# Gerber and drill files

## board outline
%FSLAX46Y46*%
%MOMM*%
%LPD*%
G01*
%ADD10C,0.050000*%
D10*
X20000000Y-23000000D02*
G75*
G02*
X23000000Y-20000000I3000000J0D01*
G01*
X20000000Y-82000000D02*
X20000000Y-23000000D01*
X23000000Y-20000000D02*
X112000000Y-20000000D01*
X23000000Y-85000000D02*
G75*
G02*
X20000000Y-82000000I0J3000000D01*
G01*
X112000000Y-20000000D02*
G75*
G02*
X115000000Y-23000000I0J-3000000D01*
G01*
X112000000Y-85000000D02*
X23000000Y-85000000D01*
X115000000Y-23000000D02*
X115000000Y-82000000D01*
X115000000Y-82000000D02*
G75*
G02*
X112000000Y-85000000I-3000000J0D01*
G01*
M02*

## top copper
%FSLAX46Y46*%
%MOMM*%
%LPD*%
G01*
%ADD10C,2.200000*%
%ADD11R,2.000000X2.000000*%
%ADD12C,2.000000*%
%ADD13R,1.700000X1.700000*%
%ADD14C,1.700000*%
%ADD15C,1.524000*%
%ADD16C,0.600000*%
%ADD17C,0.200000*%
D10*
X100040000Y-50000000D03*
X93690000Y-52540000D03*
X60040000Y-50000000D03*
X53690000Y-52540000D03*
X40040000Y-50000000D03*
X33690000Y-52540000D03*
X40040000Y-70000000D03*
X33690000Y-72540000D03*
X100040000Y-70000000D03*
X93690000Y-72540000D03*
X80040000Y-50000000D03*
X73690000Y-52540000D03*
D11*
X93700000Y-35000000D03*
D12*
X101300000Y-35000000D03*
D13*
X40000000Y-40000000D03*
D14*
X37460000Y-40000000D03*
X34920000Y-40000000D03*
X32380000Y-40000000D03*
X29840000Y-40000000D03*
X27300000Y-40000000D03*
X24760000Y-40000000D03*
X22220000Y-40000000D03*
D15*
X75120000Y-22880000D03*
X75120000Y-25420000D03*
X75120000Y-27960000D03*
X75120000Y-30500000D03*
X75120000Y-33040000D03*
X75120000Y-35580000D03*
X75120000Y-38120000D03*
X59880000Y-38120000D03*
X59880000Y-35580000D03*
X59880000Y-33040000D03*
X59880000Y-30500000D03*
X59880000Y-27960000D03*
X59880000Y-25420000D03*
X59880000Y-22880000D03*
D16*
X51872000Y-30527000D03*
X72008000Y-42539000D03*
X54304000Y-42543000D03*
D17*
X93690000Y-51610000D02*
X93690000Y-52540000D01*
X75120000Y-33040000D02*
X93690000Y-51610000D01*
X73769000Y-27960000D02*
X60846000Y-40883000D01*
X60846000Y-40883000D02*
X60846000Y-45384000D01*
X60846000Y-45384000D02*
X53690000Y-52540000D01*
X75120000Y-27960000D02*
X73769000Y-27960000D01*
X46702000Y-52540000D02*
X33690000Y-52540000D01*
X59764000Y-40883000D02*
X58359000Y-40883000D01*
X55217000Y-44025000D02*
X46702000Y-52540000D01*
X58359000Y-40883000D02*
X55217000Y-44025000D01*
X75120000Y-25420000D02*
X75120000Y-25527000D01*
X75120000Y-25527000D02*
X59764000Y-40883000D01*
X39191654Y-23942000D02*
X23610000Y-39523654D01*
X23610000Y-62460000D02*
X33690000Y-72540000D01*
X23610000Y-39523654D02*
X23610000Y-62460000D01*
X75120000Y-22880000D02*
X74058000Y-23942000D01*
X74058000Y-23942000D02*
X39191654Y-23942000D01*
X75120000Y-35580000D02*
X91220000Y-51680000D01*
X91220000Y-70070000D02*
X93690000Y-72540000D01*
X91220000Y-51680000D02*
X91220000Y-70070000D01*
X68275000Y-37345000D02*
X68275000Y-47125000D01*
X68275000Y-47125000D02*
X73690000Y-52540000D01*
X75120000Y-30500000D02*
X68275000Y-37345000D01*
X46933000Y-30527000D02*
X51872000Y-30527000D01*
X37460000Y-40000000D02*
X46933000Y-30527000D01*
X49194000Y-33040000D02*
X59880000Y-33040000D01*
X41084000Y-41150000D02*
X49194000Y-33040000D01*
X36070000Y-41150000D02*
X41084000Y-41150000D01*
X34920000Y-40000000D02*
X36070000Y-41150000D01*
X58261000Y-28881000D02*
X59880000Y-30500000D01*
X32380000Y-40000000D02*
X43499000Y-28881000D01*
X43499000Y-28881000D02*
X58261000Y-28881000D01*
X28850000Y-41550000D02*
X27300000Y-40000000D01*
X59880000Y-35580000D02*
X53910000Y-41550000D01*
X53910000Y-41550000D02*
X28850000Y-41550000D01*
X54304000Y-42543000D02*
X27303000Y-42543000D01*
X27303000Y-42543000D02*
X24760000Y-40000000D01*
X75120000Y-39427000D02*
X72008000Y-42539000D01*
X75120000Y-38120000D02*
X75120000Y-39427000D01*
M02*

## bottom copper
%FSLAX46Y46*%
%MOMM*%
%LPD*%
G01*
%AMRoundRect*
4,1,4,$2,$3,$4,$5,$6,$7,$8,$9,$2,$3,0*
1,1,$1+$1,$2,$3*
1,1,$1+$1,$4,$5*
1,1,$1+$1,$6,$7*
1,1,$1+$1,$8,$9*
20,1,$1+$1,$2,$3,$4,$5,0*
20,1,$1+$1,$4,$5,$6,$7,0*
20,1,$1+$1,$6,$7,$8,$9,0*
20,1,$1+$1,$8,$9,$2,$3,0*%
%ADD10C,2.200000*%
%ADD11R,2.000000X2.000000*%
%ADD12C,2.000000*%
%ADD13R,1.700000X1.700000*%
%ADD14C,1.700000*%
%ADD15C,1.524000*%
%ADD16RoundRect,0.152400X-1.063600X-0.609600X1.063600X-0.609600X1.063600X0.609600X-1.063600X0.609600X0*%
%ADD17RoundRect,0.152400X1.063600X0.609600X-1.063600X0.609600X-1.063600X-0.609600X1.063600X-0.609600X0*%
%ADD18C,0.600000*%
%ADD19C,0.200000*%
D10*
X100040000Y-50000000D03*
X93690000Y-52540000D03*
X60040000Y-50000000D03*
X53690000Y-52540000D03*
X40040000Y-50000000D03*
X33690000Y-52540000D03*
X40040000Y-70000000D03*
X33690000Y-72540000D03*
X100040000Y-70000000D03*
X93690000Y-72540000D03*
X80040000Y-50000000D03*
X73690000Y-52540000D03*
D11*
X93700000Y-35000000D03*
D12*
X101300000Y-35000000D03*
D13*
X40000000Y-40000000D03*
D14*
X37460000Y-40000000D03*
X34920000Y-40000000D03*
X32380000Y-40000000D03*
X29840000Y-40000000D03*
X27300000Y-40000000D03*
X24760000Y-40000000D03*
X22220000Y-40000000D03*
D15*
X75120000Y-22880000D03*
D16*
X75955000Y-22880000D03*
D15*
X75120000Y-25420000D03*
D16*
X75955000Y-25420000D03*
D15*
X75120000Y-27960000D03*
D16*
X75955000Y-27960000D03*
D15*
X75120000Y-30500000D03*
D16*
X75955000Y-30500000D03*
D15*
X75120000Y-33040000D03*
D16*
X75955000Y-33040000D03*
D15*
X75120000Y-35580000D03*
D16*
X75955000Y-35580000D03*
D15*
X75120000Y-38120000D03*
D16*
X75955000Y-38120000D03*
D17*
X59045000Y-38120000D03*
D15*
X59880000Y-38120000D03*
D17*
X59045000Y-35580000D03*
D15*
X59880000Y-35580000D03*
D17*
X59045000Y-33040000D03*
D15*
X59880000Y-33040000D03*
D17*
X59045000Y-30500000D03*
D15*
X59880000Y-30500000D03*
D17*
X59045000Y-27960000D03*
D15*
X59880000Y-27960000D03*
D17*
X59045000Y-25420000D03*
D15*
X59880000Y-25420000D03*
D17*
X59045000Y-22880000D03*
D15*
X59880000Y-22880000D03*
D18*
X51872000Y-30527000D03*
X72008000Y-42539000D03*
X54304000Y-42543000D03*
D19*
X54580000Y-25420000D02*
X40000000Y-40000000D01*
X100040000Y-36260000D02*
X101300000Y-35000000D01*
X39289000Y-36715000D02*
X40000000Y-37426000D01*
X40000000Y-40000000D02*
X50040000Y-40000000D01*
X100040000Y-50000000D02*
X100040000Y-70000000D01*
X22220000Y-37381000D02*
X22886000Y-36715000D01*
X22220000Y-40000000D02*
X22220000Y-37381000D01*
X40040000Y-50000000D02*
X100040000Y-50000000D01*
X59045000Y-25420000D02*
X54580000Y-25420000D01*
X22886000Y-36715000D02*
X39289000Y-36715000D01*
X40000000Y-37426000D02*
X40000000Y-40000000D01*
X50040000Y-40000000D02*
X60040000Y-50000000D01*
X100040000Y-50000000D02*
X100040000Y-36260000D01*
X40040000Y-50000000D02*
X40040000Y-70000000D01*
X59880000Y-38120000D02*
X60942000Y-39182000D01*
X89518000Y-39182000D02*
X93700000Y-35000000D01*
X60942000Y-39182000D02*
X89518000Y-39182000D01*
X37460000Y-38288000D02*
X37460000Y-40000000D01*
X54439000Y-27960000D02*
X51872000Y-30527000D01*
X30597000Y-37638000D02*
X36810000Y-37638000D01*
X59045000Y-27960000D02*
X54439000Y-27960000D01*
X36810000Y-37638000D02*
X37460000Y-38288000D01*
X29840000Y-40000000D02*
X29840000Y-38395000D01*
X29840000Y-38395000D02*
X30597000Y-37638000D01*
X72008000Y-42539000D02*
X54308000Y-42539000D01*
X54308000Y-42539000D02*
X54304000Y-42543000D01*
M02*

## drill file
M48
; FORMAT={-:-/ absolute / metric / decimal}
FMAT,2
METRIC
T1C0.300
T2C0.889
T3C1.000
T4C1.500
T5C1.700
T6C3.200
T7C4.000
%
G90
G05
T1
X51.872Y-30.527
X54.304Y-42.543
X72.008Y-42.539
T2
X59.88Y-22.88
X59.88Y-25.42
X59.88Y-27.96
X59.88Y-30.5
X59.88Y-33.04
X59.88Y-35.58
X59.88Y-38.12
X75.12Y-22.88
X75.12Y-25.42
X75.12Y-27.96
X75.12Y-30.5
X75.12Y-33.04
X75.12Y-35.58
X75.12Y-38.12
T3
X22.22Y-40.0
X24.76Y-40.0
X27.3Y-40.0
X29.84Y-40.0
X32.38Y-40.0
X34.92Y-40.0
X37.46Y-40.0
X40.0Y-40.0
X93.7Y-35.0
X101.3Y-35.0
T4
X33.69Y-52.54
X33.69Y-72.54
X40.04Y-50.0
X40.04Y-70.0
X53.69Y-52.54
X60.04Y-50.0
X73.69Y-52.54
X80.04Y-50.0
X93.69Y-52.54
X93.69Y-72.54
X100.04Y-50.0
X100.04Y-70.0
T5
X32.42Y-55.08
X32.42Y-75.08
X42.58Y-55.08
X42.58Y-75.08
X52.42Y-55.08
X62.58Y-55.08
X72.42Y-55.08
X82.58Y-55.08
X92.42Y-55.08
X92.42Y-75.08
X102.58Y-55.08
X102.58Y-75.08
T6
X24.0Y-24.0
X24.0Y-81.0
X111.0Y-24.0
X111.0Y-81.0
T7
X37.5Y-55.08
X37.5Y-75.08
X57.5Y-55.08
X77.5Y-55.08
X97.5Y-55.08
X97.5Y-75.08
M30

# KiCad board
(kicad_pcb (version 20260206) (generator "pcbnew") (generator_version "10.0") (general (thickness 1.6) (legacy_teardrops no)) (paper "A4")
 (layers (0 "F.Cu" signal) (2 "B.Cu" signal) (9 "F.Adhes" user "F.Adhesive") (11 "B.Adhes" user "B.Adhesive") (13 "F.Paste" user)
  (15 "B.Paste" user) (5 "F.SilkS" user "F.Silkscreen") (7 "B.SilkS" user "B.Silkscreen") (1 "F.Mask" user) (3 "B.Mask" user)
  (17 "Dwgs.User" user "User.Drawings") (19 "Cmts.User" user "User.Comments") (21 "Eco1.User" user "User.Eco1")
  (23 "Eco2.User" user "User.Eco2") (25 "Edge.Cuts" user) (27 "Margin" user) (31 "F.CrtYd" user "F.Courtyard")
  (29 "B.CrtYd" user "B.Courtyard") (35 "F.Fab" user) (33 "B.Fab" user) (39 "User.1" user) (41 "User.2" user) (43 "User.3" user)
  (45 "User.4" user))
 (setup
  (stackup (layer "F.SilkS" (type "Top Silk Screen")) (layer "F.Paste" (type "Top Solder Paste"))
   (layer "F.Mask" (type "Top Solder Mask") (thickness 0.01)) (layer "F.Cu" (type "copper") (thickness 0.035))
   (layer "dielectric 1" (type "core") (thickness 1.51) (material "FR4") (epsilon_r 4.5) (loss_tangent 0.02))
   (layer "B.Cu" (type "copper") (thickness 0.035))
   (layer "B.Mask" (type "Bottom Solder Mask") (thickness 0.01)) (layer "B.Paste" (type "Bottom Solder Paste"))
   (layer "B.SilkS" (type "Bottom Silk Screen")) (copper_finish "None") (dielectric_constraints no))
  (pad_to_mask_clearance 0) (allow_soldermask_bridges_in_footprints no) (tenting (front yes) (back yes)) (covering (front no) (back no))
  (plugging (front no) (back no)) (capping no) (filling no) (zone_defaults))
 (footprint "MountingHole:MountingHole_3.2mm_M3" (layer "F.Cu") (at 24 81)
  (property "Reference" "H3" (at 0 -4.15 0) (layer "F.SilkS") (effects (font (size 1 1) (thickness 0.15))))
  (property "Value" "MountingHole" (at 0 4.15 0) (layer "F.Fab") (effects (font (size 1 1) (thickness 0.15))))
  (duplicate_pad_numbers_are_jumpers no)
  (pad "" np_thru_hole circle (at 0 0) (size 3.2 3.2) (drill 3.2) (layers "*.Cu" "*.Mask")))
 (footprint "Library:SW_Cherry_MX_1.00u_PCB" (layer "F.Cu") (at 100.04 50)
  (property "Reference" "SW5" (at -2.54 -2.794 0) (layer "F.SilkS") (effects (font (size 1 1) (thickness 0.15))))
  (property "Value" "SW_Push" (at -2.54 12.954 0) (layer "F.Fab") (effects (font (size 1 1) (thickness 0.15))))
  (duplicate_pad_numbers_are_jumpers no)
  (pad "" np_thru_hole circle (at -7.62 5.08) (size 1.7 1.7) (drill 1.7) (layers "*.Cu" "*.Mask"))
  (pad "" np_thru_hole circle (at -2.54 5.08) (size 4 4) (drill 4) (layers "*.Cu" "*.Mask"))
  (pad "" np_thru_hole circle (at 2.54 5.08) (size 1.7 1.7) (drill 1.7) (layers "*.Cu" "*.Mask"))
  (pad "1" thru_hole circle (at 0 0) (size 2.2 2.2) (drill 1.5) (layers "*.Cu" "*.Mask") (remove_unused_layers no) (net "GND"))
  (pad "2" thru_hole circle (at -6.35 2.54) (size 2.2 2.2) (drill 1.5) (layers "*.Cu" "*.Mask") (remove_unused_layers no)
   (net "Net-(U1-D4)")))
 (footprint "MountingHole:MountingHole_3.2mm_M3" (layer "F.Cu") (at 111 81)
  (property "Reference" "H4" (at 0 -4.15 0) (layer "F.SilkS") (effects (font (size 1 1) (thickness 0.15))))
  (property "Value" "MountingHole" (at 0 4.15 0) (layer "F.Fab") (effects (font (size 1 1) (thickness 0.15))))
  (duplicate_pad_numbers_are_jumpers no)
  (pad "" np_thru_hole circle (at 0 0) (size 3.2 3.2) (drill 3.2) (layers "*.Cu" "*.Mask")))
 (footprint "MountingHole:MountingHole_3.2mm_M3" (layer "F.Cu") (at 111 24 180)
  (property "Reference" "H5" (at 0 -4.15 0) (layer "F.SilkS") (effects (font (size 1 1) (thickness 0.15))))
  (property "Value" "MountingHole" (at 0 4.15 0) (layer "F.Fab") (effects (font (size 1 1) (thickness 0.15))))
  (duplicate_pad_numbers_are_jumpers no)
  (pad "" np_thru_hole circle (at 0 0 180) (size 3.2 3.2) (drill 3.2) (layers "*.Cu" "*.Mask")))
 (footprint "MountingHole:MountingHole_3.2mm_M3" (layer "F.Cu") (at 24 24 180)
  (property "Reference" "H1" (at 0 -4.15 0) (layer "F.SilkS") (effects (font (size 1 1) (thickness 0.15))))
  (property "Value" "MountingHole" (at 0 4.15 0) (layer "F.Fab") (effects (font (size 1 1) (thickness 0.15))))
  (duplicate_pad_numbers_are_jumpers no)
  (pad "" np_thru_hole circle (at 0 0 180) (size 3.2 3.2) (drill 3.2) (layers "*.Cu" "*.Mask")))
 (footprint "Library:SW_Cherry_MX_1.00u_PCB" (layer "F.Cu") (at 60.04 50)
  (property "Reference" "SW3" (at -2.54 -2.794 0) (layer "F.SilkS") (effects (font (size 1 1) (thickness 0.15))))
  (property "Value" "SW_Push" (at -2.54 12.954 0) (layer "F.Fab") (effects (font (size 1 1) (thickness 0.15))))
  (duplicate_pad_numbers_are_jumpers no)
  (pad "" np_thru_hole circle (at -7.62 5.08) (size 1.7 1.7) (drill 1.7) (layers "*.Cu" "*.Mask"))
  (pad "" np_thru_hole circle (at -2.54 5.08) (size 4 4) (drill 4) (layers "*.Cu" "*.Mask"))
  (pad "" np_thru_hole circle (at 2.54 5.08) (size 1.7 1.7) (drill 1.7) (layers "*.Cu" "*.Mask"))
  (pad "1" thru_hole circle (at 0 0) (size 2.2 2.2) (drill 1.5) (layers "*.Cu" "*.Mask") (remove_unused_layers no) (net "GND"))
  (pad "2" thru_hole circle (at -6.35 2.54) (size 2.2 2.2) (drill 1.5) (layers "*.Cu" "*.Mask") (remove_unused_layers no)
   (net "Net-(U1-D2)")))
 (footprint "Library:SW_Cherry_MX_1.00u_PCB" (layer "F.Cu") (at 40.04 50)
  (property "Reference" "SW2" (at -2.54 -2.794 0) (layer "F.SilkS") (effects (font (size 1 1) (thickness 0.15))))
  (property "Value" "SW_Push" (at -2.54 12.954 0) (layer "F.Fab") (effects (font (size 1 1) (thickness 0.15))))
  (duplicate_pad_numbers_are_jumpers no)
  (pad "" np_thru_hole circle (at -7.62 5.08) (size 1.7 1.7) (drill 1.7) (layers "*.Cu" "*.Mask"))
  (pad "" np_thru_hole circle (at -2.54 5.08) (size 4 4) (drill 4) (layers "*.Cu" "*.Mask"))
  (pad "" np_thru_hole circle (at 2.54 5.08) (size 1.7 1.7) (drill 1.7) (layers "*.Cu" "*.Mask"))
  (pad "1" thru_hole circle (at 0 0) (size 2.2 2.2) (drill 1.5) (layers "*.Cu" "*.Mask") (remove_unused_layers no) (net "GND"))
  (pad "2" thru_hole circle (at -6.35 2.54) (size 2.2 2.2) (drill 1.5) (layers "*.Cu" "*.Mask") (remove_unused_layers no)
   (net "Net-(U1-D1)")))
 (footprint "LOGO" (layer "F.Cu") (at 40 28)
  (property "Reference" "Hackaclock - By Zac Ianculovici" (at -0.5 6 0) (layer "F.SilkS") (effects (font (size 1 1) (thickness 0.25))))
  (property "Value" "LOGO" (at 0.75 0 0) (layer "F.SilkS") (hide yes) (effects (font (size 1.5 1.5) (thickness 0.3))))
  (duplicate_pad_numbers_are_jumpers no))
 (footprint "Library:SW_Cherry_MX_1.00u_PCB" (layer "F.Cu") (at 40.04 70)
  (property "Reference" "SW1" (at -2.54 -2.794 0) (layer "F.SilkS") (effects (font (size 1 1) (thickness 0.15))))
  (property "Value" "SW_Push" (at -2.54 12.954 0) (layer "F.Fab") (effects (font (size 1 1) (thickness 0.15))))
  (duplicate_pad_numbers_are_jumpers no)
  (pad "" np_thru_hole circle (at -7.62 5.08) (size 1.7 1.7) (drill 1.7) (layers "*.Cu" "*.Mask"))
  (pad "" np_thru_hole circle (at -2.54 5.08) (size 4 4) (drill 4) (layers "*.Cu" "*.Mask"))
  (pad "" np_thru_hole circle (at 2.54 5.08) (size 1.7 1.7) (drill 1.7) (layers "*.Cu" "*.Mask"))
  (pad "1" thru_hole circle (at 0 0) (size 2.2 2.2) (drill 1.5) (layers "*.Cu" "*.Mask") (remove_unused_layers no) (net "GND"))
  (pad "2" thru_hole circle (at -6.35 2.54) (size 2.2 2.2) (drill 1.5) (layers "*.Cu" "*.Mask") (remove_unused_layers no)
   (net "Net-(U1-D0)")))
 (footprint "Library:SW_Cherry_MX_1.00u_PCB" (layer "F.Cu") (at 100.04 70)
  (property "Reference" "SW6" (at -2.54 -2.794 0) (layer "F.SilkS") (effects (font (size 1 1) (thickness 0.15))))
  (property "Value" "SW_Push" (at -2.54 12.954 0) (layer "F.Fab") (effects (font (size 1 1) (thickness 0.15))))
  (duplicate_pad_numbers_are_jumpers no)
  (pad "" np_thru_hole circle (at -7.62 5.08) (size 1.7 1.7) (drill 1.7) (layers "*.Cu" "*.Mask"))
  (pad "" np_thru_hole circle (at -2.54 5.08) (size 4 4) (drill 4) (layers "*.Cu" "*.Mask"))
  (pad "" np_thru_hole circle (at 2.54 5.08) (size 1.7 1.7) (drill 1.7) (layers "*.Cu" "*.Mask"))
  (pad "1" thru_hole circle (at 0 0) (size 2.2 2.2) (drill 1.5) (layers "*.Cu" "*.Mask") (remove_unused_layers no) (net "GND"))
  (pad "2" thru_hole circle (at -6.35 2.54) (size 2.2 2.2) (drill 1.5) (layers "*.Cu" "*.Mask") (remove_unused_layers no)
   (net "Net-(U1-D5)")))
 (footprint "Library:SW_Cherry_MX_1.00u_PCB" (layer "F.Cu") (at 80.04 50)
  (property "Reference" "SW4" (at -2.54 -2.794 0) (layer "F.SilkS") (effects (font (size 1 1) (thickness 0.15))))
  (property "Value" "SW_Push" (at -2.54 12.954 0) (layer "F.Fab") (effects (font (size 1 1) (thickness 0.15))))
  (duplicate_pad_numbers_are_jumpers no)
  (pad "" np_thru_hole circle (at -7.62 5.08) (size 1.7 1.7) (drill 1.7) (layers "*.Cu" "*.Mask"))
  (pad "" np_thru_hole circle (at -2.54 5.08) (size 4 4) (drill 4) (layers "*.Cu" "*.Mask"))
  (pad "" np_thru_hole circle (at 2.54 5.08) (size 1.7 1.7) (drill 1.7) (layers "*.Cu" "*.Mask"))
  (pad "1" thru_hole circle (at 0 0) (size 2.2 2.2) (drill 1.5) (layers "*.Cu" "*.Mask") (remove_unused_layers no) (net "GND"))
  (pad "2" thru_hole circle (at -6.35 2.54) (size 2.2 2.2) (drill 1.5) (layers "*.Cu" "*.Mask") (remove_unused_layers no)
   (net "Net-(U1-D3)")))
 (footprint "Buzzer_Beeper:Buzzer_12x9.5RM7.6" (layer "B.Cu") (at 93.7 35)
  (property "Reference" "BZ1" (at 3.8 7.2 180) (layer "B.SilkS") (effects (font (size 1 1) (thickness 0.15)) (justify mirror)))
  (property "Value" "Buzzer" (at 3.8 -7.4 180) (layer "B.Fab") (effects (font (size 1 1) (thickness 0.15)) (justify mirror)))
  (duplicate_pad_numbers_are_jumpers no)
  (pad "1" thru_hole rect (at 0 0) (size 2 2) (drill 1) (layers "*.Cu" "*.Mask") (remove_unused_layers no) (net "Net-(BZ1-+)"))
  (pad "2" thru_hole circle (at 7.6 0) (size 2 2) (drill 1) (layers "*.Cu" "*.Mask") (remove_unused_layers no) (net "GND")))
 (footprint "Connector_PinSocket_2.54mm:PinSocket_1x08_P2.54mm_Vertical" (layer "B.Cu") (at 40 40 90)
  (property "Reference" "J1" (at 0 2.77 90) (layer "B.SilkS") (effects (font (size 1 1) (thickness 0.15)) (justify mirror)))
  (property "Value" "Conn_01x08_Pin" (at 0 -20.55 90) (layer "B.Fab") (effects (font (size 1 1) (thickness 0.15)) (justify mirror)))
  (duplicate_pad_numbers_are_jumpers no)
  (pad "1" thru_hole rect (at 0 0 90) (size 1.7 1.7) (drill 1) (layers "*.Cu" "*.Mask") (remove_unused_layers no) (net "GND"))
  (pad "2" thru_hole circle (at 0 -2.54 90) (size 1.7 1.7) (drill 1) (layers "*.Cu" "*.Mask") (remove_unused_layers no) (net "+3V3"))
  (pad "3" thru_hole circle (at 0 -5.08 90) (size 1.7 1.7) (drill 1) (layers "*.Cu" "*.Mask") (remove_unused_layers no) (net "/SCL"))
  (pad "4" thru_hole circle (at 0 -7.62 90) (size 1.7 1.7) (drill 1) (layers "*.Cu" "*.Mask") (remove_unused_layers no) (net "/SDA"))
  (pad "5" thru_hole circle (at 0 -10.16 90) (size 1.7 1.7) (drill 1) (layers "*.Cu" "*.Mask") (remove_unused_layers no) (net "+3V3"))
  (pad "6" thru_hole circle (at 0 -12.7 90) (size 1.7 1.7) (drill 1) (layers "*.Cu" "*.Mask") (remove_unused_layers no) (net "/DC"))
  (pad "7" thru_hole circle (at 0 -15.24 90) (size 1.7 1.7) (drill 1) (layers "*.Cu" "*.Mask") (remove_unused_layers no) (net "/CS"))
  (pad "8" thru_hole circle (at 0 -17.78 90) (size 1.7 1.7) (drill 1) (layers "*.Cu" "*.Mask") (remove_unused_layers no) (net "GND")))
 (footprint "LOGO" (layer "B.Cu") (at 40 28 180)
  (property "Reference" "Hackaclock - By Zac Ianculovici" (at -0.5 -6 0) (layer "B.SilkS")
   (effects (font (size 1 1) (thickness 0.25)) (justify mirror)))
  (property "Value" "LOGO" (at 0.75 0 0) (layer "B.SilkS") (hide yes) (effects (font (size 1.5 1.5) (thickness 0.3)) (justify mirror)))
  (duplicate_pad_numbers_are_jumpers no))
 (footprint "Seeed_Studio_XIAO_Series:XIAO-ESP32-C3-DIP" (layer "B.Cu") (at 67.5 30.5 90)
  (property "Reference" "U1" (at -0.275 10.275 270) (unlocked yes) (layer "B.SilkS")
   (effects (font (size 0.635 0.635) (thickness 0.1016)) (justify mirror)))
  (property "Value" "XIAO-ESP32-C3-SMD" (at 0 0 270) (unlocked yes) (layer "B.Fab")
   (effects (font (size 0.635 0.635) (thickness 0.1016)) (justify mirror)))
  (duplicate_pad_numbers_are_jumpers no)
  (pad "1" thru_hole circle (at 7.62 7.62) (size 1.524 1.524) (drill 0.889) (layers "*.Cu" "*.Mask") (remove_unused_layers no)
   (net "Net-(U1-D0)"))
  (pad "1" smd roundrect (at 7.62 8.455) (size 2.432 1.524) (layers "B.Cu" "B.Mask") (roundrect_rratio 0.1) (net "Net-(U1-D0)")
   (thermal_bridge_angle 45))
  (pad "2" thru_hole circle (at 5.08 7.62) (size 1.524 1.524) (drill 0.889) (layers "*.Cu" "*.Mask") (remove_unused_layers no)
   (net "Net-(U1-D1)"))
  (pad "2" smd roundrect (at 5.08 8.455) (size 2.432 1.524) (layers "B.Cu" "B.Mask") (roundrect_rratio 0.1) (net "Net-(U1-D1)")
   (thermal_bridge_angle 45))
  (pad "3" thru_hole circle (at 2.54 7.62) (size 1.524 1.524) (drill 0.889) (layers "*.Cu" "*.Mask") (remove_unused_layers no)
   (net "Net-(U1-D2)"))
  (pad "3" smd roundrect (at 2.54 8.455) (size 2.432 1.524) (layers "B.Cu" "B.Mask") (roundrect_rratio 0.1) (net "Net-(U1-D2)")
   (thermal_bridge_angle 45))
  (pad "4" thru_hole circle (at 0 7.62) (size 1.524 1.524) (drill 0.889) (layers "*.Cu" "*.Mask") (remove_unused_layers no)
   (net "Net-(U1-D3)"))
  (pad "4" smd roundrect (at 0 8.455) (size 2.432 1.524) (layers "B.Cu" "B.Mask") (roundrect_rratio 0.1) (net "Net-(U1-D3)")
   (thermal_bridge_angle 45))
  (pad "5" thru_hole circle (at -2.54 7.62) (size 1.524 1.524) (drill 0.889) (layers "*.Cu" "*.Mask") (remove_unused_layers no)
   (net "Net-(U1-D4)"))
  (pad "5" smd roundrect (at -2.54 8.455) (size 2.432 1.524) (layers "B.Cu" "B.Mask") (roundrect_rratio 0.1) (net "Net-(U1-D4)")
   (thermal_bridge_angle 45))
  (pad "6" thru_hole circle (at -5.08 7.62) (size 1.524 1.524) (drill 0.889) (layers "*.Cu" "*.Mask") (remove_unused_layers no)
   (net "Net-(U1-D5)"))
  (pad "6" smd roundrect (at -5.08 8.455) (size 2.432 1.524) (layers "B.Cu" "B.Mask") (roundrect_rratio 0.1) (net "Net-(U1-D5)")
   (thermal_bridge_angle 45))
  (pad "7" thru_hole circle (at -7.62 7.62) (size 1.524 1.524) (drill 0.889) (layers "*.Cu" "*.Mask") (remove_unused_layers no) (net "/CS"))
  (pad "7" smd roundrect (at -7.62 8.455) (size 2.432 1.524) (layers "B.Cu" "B.Mask") (roundrect_rratio 0.1) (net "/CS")
   (thermal_bridge_angle 45))
  (pad "8" smd roundrect (at -7.62 -8.455 180) (size 2.432 1.524) (layers "B.Cu" "B.Mask") (roundrect_rratio 0.1) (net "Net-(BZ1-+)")
   (thermal_bridge_angle 45))
  (pad "8" thru_hole circle (at -7.62 -7.62 180) (size 1.524 1.524) (drill 0.889) (layers "*.Cu" "*.Mask") (remove_unused_layers no)
   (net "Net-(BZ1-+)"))
  (pad "9" smd roundrect (at -5.08 -8.455 180) (size 2.432 1.524) (layers "B.Cu" "B.Mask") (roundrect_rratio 0.1) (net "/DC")
   (thermal_bridge_angle 45))
  (pad "9" thru_hole circle (at -5.08 -7.62 180) (size 1.524 1.524) (drill 0.889) (layers "*.Cu" "*.Mask") (remove_unused_layers no)
   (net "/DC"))
  (pad "10" smd roundrect (at -2.54 -8.455 180) (size 2.432 1.524) (layers "B.Cu" "B.Mask") (roundrect_rratio 0.1) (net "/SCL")
   (thermal_bridge_angle 45))
  (pad "10" thru_hole circle (at -2.54 -7.62 180) (size 1.524 1.524) (drill 0.889) (layers "*.Cu" "*.Mask") (remove_unused_layers no)
   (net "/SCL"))
  (pad "11" smd roundrect (at 0 -8.455 180) (size 2.432 1.524) (layers "B.Cu" "B.Mask") (roundrect_rratio 0.1) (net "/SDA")
   (thermal_bridge_angle 45))
  (pad "11" thru_hole circle (at 0 -7.62 180) (size 1.524 1.524) (drill 0.889) (layers "*.Cu" "*.Mask") (remove_unused_layers no)
   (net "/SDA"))
  (pad "12" smd roundrect (at 2.54 -8.455 180) (size 2.432 1.524) (layers "B.Cu" "B.Mask") (roundrect_rratio 0.1) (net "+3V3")
   (thermal_bridge_angle 45))
  (pad "12" thru_hole circle (at 2.54 -7.62 180) (size 1.524 1.524) (drill 0.889) (layers "*.Cu" "*.Mask") (remove_unused_layers no)
   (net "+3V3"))
  (pad "13" smd roundrect (at 5.08 -8.455 180) (size 2.432 1.524) (layers "B.Cu" "B.Mask") (roundrect_rratio 0.1) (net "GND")
   (thermal_bridge_angle 45))
  (pad "13" thru_hole circle (at 5.08 -7.62 180) (size 1.524 1.524) (drill 0.889) (layers "*.Cu" "*.Mask") (remove_unused_layers no)
   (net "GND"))
  (pad "14" smd roundrect (at 7.62 -8.455 180) (size 2.432 1.524) (layers "B.Cu" "B.Mask") (roundrect_rratio 0.1)
   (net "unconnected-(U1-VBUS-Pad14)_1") (thermal_bridge_angle 45))
  (pad "14" thru_hole circle (at 7.62 -7.62 180) (size 1.524 1.524) (drill 0.889) (layers "*.Cu" "*.Mask") (remove_unused_layers no)
   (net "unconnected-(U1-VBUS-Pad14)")))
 (gr_arc (start 20 23) (mid 20.87868 20.87868) (end 23 20) (stroke (width 0.05) (type default)) (layer "Edge.Cuts"))
 (gr_line (start 20 82) (end 20 23) (stroke (width 0.05) (type default)) (layer "Edge.Cuts"))
 (gr_line (start 23 20) (end 112 20) (stroke (width 0.05) (type default)) (layer "Edge.Cuts"))
 (gr_arc (start 23 85) (mid 20.87868 84.12132) (end 20 82) (stroke (width 0.05) (type default)) (layer "Edge.Cuts"))
 (gr_arc (start 112 20) (mid 114.12132 20.87868) (end 115 23) (stroke (width 0.05) (type default)) (layer "Edge.Cuts"))
 (gr_line (start 112 85) (end 23 85) (stroke (width 0.05) (type default)) (layer "Edge.Cuts"))
 (gr_line (start 115 23) (end 115 82) (stroke (width 0.05) (type default)) (layer "Edge.Cuts"))
 (gr_arc (start 115 82) (mid 114.12132 84.12132) (end 112 85) (stroke (width 0.05) (type default)) (layer "Edge.Cuts"))
 (segment (start 54.58 25.42) (end 40 40) (width 0.2) (layer "B.Cu") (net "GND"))
 (segment (start 100.04 36.26) (end 101.3 35) (width 0.2) (layer "B.Cu") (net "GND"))
 (segment (start 39.289 36.715) (end 40 37.426) (width 0.2) (layer "B.Cu") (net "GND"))
 (segment (start 40 40) (end 50.04 40) (width 0.2) (layer "B.Cu") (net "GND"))
 (segment (start 100.04 50) (end 100.04 70) (width 0.2) (layer "B.Cu") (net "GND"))
 (segment (start 22.22 37.381) (end 22.886 36.715) (width 0.2) (layer "B.Cu") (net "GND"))
 (segment (start 22.22 40) (end 22.22 37.381) (width 0.2) (layer "B.Cu") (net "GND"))
 (segment (start 40.04 50) (end 100.04 50) (width 0.2) (layer "B.Cu") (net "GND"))
 (segment (start 59.045 25.42) (end 54.58 25.42) (width 0.2) (layer "B.Cu") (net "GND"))
 (segment (start 22.886 36.715) (end 39.289 36.715) (width 0.2) (layer "B.Cu") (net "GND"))
 (segment (start 40 37.426) (end 40 40) (width 0.2) (layer "B.Cu") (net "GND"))
 (segment (start 50.04 40) (end 60.04 50) (width 0.2) (layer "B.Cu") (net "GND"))
 (segment (start 100.04 50) (end 100.04 36.26) (width 0.2) (layer "B.Cu") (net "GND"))
 (segment (start 40.04 50) (end 40.04 70) (width 0.2) (layer "B.Cu") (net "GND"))
 (segment (start 93.69 51.61) (end 93.69 52.54) (width 0.2) (layer "F.Cu") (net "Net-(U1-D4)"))
 (segment (start 75.12 33.04) (end 93.69 51.61) (width 0.2) (layer "F.Cu") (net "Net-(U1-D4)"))
 (segment (start 73.769 27.96) (end 60.846 40.883) (width 0.2) (layer "F.Cu") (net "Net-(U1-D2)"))
 (segment (start 60.846 40.883) (end 60.846 45.384) (width 0.2) (layer "F.Cu") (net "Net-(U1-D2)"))
 (segment (start 60.846 45.384) (end 53.69 52.54) (width 0.2) (layer "F.Cu") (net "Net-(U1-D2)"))
 (segment (start 75.12 27.96) (end 73.769 27.96) (width 0.2) (layer "F.Cu") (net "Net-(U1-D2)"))
 (segment (start 46.702 52.54) (end 33.69 52.54) (width 0.2) (layer "F.Cu") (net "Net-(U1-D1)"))
 (segment (start 59.764 40.883) (end 58.359 40.883) (width 0.2) (layer "F.Cu") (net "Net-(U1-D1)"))
 (segment (start 55.217 44.025) (end 46.702 52.54) (width 0.2) (layer "F.Cu") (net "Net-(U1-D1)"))
 (segment (start 58.359 40.883) (end 55.217 44.025) (width 0.2) (layer "F.Cu") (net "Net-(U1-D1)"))
 (segment (start 75.12 25.42) (end 75.12 25.527) (width 0.2) (layer "F.Cu") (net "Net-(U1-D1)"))
 (segment (start 75.12 25.527) (end 59.764 40.883) (width 0.2) (layer "F.Cu") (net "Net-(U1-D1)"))
 (segment (start 39.191654 23.942) (end 23.61 39.523654) (width 0.2) (layer "F.Cu") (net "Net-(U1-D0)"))
 (segment (start 23.61 62.46) (end 33.69 72.54) (width 0.2) (layer "F.Cu") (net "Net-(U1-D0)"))
 (segment (start 23.61 39.523654) (end 23.61 62.46) (width 0.2) (layer "F.Cu") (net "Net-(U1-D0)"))
 (segment (start 75.12 22.88) (end 74.058 23.942) (width 0.2) (layer "F.Cu") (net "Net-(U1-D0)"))
 (segment (start 74.058 23.942) (end 39.191654 23.942) (width 0.2) (layer "F.Cu") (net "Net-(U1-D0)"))
 (segment (start 75.12 35.58) (end 91.22 51.68) (width 0.2) (layer "F.Cu") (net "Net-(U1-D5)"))
 (segment (start 91.22 70.07) (end 93.69 72.54) (width 0.2) (layer "F.Cu") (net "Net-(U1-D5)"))
 (segment (start 91.22 51.68) (end 91.22 70.07) (width 0.2) (layer "F.Cu") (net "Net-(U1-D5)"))
 (segment (start 68.275 37.345) (end 68.275 47.125) (width 0.2) (layer "F.Cu") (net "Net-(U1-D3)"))
 (segment (start 68.275 47.125) (end 73.69 52.54) (width 0.2) (layer "F.Cu") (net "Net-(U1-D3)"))
 (segment (start 75.12 30.5) (end 68.275 37.345) (width 0.2) (layer "F.Cu") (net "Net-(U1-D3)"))
 (segment (start 59.88 38.12) (end 60.942 39.182) (width 0.2) (layer "B.Cu") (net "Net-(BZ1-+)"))
 (segment (start 89.518 39.182) (end 93.7 35) (width 0.2) (layer "B.Cu") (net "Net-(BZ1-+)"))
 (segment (start 60.942 39.182) (end 89.518 39.182) (width 0.2) (layer "B.Cu") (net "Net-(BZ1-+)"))
 (segment (start 46.933 30.527) (end 51.872 30.527) (width 0.2) (layer "F.Cu") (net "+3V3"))
 (segment (start 37.46 40) (end 46.933 30.527) (width 0.2) (layer "F.Cu") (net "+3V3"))
 (via (at 51.872 30.527) (size 0.6) (drill 0.3) (layers "F.Cu" "B.Cu") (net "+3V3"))
 (segment (start 37.46 38.288) (end 37.46 40) (width 0.2) (layer "B.Cu") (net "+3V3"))
 (segment (start 54.439 27.96) (end 51.872 30.527) (width 0.2) (layer "B.Cu") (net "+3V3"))
 (segment (start 30.597 37.638) (end 36.81 37.638) (width 0.2) (layer "B.Cu") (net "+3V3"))
 (segment (start 59.045 27.96) (end 54.439 27.96) (width 0.2) (layer "B.Cu") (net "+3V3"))
 (segment (start 36.81 37.638) (end 37.46 38.288) (width 0.2) (layer "B.Cu") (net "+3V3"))
 (segment (start 29.84 40) (end 29.84 38.395) (width 0.2) (layer "B.Cu") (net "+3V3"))
 (segment (start 29.84 38.395) (end 30.597 37.638) (width 0.2) (layer "B.Cu") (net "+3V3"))
 (segment (start 49.194 33.04) (end 59.88 33.04) (width 0.2) (layer "F.Cu") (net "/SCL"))
 (segment (start 41.084 41.15) (end 49.194 33.04) (width 0.2) (layer "F.Cu") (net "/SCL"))
 (segment (start 36.07 41.15) (end 41.084 41.15) (width 0.2) (layer "F.Cu") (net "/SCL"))
 (segment (start 34.92 40) (end 36.07 41.15) (width 0.2) (layer "F.Cu") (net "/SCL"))
 (segment (start 58.261 28.881) (end 59.88 30.5) (width 0.2) (layer "F.Cu") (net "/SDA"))
 (segment (start 32.38 40) (end 43.499 28.881) (width 0.2) (layer "F.Cu") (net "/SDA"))
 (segment (start 43.499 28.881) (end 58.261 28.881) (width 0.2) (layer "F.Cu") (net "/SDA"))
 (segment (start 28.85 41.55) (end 27.3 40) (width 0.2) (layer "F.Cu") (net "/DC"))
 (segment (start 59.88 35.58) (end 53.91 41.55) (width 0.2) (layer "F.Cu") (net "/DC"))
 (segment (start 53.91 41.55) (end 28.85 41.55) (width 0.2) (layer "F.Cu") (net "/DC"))
 (segment (start 54.304 42.543) (end 27.303 42.543) (width 0.2) (layer "F.Cu") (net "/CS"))
 (segment (start 27.303 42.543) (end 24.76 40) (width 0.2) (layer "F.Cu") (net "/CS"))
 (segment (start 75.12 39.427) (end 72.008 42.539) (width 0.2) (layer "F.Cu") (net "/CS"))
 (segment (start 75.12 38.12) (end 75.12 39.427) (width 0.2) (layer "F.Cu") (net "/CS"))
 (via (at 72.008 42.539) (size 0.6) (drill 0.3) (layers "F.Cu" "B.Cu") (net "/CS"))
 (via (at 54.304 42.543) (size 0.6) (drill 0.3) (layers "F.Cu" "B.Cu") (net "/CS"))
 (segment (start 72.008 42.539) (end 54.308 42.539) (width 0.2) (layer "B.Cu") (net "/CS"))
 (segment (start 54.308 42.539) (end 54.304 42.543) (width 0.2) (layer "B.Cu") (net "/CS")))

